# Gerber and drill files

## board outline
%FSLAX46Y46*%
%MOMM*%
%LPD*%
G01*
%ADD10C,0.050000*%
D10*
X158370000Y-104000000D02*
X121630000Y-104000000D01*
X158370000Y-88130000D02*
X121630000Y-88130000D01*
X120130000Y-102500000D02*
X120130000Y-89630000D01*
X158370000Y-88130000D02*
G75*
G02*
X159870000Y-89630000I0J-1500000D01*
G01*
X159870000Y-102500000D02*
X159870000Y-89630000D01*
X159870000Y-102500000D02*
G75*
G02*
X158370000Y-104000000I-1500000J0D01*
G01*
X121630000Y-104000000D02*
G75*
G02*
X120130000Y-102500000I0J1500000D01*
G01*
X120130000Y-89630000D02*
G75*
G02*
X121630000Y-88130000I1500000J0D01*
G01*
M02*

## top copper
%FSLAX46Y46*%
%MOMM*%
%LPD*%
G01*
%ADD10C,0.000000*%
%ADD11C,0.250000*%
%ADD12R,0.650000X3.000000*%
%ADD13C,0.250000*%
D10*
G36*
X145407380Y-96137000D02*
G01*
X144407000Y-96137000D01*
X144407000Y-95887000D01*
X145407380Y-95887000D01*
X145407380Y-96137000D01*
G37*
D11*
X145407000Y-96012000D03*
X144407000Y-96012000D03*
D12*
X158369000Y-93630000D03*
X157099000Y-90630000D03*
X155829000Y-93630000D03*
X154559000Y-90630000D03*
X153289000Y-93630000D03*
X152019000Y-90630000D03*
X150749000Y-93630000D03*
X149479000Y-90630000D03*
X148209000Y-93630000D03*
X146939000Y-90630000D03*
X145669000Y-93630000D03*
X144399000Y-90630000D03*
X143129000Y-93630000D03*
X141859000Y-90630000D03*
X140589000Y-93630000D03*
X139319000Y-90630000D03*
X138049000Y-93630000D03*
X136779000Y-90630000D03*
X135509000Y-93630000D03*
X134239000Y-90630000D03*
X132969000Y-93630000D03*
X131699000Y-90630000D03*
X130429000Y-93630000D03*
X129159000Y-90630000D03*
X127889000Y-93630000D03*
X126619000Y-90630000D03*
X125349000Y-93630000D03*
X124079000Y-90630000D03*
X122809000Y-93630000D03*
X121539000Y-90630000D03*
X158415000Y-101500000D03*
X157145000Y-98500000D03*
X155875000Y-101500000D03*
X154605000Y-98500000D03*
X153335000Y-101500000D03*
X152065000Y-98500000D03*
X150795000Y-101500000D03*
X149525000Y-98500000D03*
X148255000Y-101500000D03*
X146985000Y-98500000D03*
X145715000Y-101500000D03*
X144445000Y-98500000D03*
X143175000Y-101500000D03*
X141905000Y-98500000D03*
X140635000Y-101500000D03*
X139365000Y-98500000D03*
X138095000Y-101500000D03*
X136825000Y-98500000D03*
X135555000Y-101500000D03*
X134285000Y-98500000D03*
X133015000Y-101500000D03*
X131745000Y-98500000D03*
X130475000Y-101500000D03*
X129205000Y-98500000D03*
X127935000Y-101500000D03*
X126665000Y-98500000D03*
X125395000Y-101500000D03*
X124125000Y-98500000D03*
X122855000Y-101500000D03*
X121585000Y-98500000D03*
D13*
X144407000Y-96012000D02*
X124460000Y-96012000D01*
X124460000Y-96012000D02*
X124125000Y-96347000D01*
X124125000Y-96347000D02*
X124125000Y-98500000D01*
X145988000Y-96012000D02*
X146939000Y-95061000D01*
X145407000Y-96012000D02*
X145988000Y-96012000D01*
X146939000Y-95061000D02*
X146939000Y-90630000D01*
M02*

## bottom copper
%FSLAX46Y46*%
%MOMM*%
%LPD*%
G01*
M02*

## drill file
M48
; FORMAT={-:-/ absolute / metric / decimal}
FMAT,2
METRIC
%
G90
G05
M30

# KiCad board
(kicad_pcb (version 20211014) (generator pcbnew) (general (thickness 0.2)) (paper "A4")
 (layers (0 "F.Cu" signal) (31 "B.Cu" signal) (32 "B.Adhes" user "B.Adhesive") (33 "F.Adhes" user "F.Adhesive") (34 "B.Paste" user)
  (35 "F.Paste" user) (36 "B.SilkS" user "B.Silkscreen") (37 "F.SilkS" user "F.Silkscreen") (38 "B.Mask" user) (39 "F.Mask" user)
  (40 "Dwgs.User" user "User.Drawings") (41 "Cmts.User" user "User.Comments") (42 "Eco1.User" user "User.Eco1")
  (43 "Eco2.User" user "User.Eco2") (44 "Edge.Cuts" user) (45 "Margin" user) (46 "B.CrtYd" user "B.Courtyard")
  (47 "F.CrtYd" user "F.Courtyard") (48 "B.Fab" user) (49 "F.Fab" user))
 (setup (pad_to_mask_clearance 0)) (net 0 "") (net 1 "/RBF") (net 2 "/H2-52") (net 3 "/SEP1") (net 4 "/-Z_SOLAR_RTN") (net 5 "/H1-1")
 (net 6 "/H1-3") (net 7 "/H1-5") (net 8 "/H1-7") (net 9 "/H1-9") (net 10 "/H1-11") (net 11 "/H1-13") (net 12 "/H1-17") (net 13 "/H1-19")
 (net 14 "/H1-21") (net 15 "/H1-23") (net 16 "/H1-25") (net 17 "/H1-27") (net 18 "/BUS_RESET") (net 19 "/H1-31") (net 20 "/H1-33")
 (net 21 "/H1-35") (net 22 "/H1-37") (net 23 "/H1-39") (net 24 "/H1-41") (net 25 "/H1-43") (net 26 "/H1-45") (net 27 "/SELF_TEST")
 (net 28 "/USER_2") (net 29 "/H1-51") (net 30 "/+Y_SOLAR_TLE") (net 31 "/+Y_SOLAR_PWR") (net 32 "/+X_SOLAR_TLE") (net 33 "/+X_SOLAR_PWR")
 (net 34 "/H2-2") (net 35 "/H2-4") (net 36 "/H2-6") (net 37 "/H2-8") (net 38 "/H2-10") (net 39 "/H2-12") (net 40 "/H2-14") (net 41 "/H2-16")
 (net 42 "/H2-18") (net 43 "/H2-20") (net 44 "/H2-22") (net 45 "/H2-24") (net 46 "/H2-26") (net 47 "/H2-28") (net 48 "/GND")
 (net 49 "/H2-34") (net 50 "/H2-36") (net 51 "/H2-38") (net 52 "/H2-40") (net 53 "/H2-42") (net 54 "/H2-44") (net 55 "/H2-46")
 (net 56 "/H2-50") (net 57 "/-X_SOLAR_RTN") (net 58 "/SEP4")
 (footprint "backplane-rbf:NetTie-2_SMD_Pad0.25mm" (layer "F.Cu") (at 144.907 96.012 180)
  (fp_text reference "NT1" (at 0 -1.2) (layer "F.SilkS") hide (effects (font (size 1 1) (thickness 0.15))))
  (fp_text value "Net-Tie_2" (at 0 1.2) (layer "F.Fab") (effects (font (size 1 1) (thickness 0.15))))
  (fp_poly (pts (xy -0.50038 -0.125) (xy 0.5 -0.125) (xy 0.5 0.125) (xy -0.50038 0.125)) (layer "F.Cu") (width 0) (fill solid))
  (pad "1" smd circle locked (at -0.5 0 180) (size 0.25 0.25) (layers "F.Cu") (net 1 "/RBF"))
  (pad "2" smd circle locked (at 0.5 0 180) (size 0.25 0.25) (layers "F.Cu") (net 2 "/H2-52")))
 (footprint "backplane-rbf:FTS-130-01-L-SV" (layer "F.Cu") (at 139.954 92.13 -90)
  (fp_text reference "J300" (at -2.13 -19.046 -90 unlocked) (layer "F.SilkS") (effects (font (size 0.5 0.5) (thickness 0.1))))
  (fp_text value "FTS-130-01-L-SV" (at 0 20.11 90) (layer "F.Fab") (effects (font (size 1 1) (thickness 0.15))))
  (pad "1" smd rect locked (at 1.5 -18.415 270) (size 3 0.65) (layers "F.Cu" "F.Paste" "F.Mask") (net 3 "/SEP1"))
  (pad "2" smd rect locked (at -1.5 -17.145 270) (size 3 0.65) (layers "F.Cu" "F.Paste" "F.Mask") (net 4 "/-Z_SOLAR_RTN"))
  (pad "3" smd rect locked (at 1.5 -15.875 270) (size 3 0.65) (layers "F.Cu" "F.Paste" "F.Mask") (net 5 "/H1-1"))
  (pad "4" smd rect locked (at -1.5 -14.605 270) (size 3 0.65) (layers "F.Cu" "F.Paste" "F.Mask") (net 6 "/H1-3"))
  (pad "5" smd rect locked (at 1.5 -13.335 270) (size 3 0.65) (layers "F.Cu" "F.Paste" "F.Mask") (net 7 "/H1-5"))
  (pad "6" smd rect locked (at -1.5 -12.065 270) (size 3 0.65) (layers "F.Cu" "F.Paste" "F.Mask") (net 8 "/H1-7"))
  (pad "7" smd rect locked (at 1.5 -10.795 270) (size 3 0.65) (layers "F.Cu" "F.Paste" "F.Mask") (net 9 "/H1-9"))
  (pad "8" smd rect locked (at -1.5 -9.525 270) (size 3 0.65) (layers "F.Cu" "F.Paste" "F.Mask") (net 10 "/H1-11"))
  (pad "9" smd rect locked (at 1.5 -8.255 270) (size 3 0.65) (layers "F.Cu" "F.Paste" "F.Mask") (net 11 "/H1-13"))
  (pad "10" smd rect locked (at -1.5 -6.985 270) (size 3 0.65) (layers "F.Cu" "F.Paste" "F.Mask") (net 1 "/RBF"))
  (pad "11" smd rect locked (at 1.5 -5.715 270) (size 3 0.65) (layers "F.Cu" "F.Paste" "F.Mask") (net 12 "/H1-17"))
  (pad "12" smd rect locked (at -1.5 -4.445 270) (size 3 0.65) (layers "F.Cu" "F.Paste" "F.Mask") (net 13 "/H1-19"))
  (pad "13" smd rect locked (at 1.5 -3.175 270) (size 3 0.65) (layers "F.Cu" "F.Paste" "F.Mask") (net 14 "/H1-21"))
  (pad "14" smd rect locked (at -1.5 -1.905 270) (size 3 0.65) (layers "F.Cu" "F.Paste" "F.Mask") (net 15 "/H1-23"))
  (pad "15" smd rect locked (at 1.5 -0.635 270) (size 3 0.65) (layers "F.Cu" "F.Paste" "F.Mask") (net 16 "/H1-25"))
  (pad "16" smd rect locked (at -1.5 0.635 270) (size 3 0.65) (layers "F.Cu" "F.Paste" "F.Mask") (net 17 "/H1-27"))
  (pad "17" smd rect locked (at 1.5 1.905 270) (size 3 0.65) (layers "F.Cu" "F.Paste" "F.Mask") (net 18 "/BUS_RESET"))
  (pad "18" smd rect locked (at -1.5 3.175 270) (size 3 0.65) (layers "F.Cu" "F.Paste" "F.Mask") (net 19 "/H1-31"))
  (pad "19" smd rect locked (at 1.5 4.445 270) (size 3 0.65) (layers "F.Cu" "F.Paste" "F.Mask") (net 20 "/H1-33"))
  (pad "20" smd rect locked (at -1.5 5.715 270) (size 3 0.65) (layers "F.Cu" "F.Paste" "F.Mask") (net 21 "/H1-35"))
  (pad "21" smd rect locked (at 1.5 6.985 270) (size 3 0.65) (layers "F.Cu" "F.Paste" "F.Mask") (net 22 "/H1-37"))
  (pad "22" smd rect locked (at -1.5 8.255 270) (size 3 0.65) (layers "F.Cu" "F.Paste" "F.Mask") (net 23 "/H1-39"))
  (pad "23" smd rect locked (at 1.5 9.525 270) (size 3 0.65) (layers "F.Cu" "F.Paste" "F.Mask") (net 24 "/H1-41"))
  (pad "24" smd rect locked (at -1.5 10.795 270) (size 3 0.65) (layers "F.Cu" "F.Paste" "F.Mask") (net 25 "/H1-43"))
  (pad "25" smd rect locked (at 1.5 12.065 270) (size 3 0.65) (layers "F.Cu" "F.Paste" "F.Mask") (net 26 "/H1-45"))
  (pad "26" smd rect locked (at -1.5 13.335 270) (size 3 0.65) (layers "F.Cu" "F.Paste" "F.Mask") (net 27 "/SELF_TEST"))
  (pad "27" smd rect locked (at 1.5 14.605 270) (size 3 0.65) (layers "F.Cu" "F.Paste" "F.Mask") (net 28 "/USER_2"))
  (pad "28" smd rect locked (at -1.5 15.875 270) (size 3 0.65) (layers "F.Cu" "F.Paste" "F.Mask") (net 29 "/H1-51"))
  (pad "29" smd rect locked (at 1.5 17.145 270) (size 3 0.65) (layers "F.Cu" "F.Paste" "F.Mask") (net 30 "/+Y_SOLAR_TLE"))
  (pad "30" smd rect locked (at -1.5 18.415 270) (size 3 0.65) (layers "F.Cu" "F.Paste" "F.Mask") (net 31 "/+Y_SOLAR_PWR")))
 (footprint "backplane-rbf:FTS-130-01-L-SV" (layer "F.Cu") (at 140 100 -90)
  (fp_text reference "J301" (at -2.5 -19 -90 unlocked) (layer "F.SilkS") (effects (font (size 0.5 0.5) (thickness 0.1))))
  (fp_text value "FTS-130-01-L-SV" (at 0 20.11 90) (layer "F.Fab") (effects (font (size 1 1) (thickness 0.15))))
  (pad "1" smd rect locked (at 1.5 -18.415 270) (size 3 0.65) (layers "F.Cu" "F.Paste" "F.Mask") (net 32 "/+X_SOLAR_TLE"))
  (pad "2" smd rect locked (at -1.5 -17.145 270) (size 3 0.65) (layers "F.Cu" "F.Paste" "F.Mask") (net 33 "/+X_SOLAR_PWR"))
  (pad "3" smd rect locked (at 1.5 -15.875 270) (size 3 0.65) (layers "F.Cu" "F.Paste" "F.Mask") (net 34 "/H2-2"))
  (pad "4" smd rect locked (at -1.5 -14.605 270) (size 3 0.65) (layers "F.Cu" "F.Paste" "F.Mask") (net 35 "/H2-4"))
  (pad "5" smd rect locked (at 1.5 -13.335 270) (size 3 0.65) (layers "F.Cu" "F.Paste" "F.Mask") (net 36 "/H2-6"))
  (pad "6" smd rect locked (at -1.5 -12.065 270) (size 3 0.65) (layers "F.Cu" "F.Paste" "F.Mask") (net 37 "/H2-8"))
  (pad "7" smd rect locked (at 1.5 -10.795 270) (size 3 0.65) (layers "F.Cu" "F.Paste" "F.Mask") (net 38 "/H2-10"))
  (pad "8" smd rect locked (at -1.5 -9.525 270) (size 3 0.65) (layers "F.Cu" "F.Paste" "F.Mask") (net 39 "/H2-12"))
  (pad "9" smd rect locked (at 1.5 -8.255 270) (size 3 0.65) (layers "F.Cu" "F.Paste" "F.Mask") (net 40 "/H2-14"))
  (pad "10" smd rect locked (at -1.5 -6.985 270) (size 3 0.65) (layers "F.Cu" "F.Paste" "F.Mask") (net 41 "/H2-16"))
  (pad "11" smd rect locked (at 1.5 -5.715 270) (size 3 0.65) (layers "F.Cu" "F.Paste" "F.Mask") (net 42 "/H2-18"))
  (pad "12" smd rect locked (at -1.5 -4.445 270) (size 3 0.65) (layers "F.Cu" "F.Paste" "F.Mask") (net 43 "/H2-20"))
  (pad "13" smd rect locked (at 1.5 -3.175 270) (size 3 0.65) (layers "F.Cu" "F.Paste" "F.Mask") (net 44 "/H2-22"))
  (pad "14" smd rect locked (at -1.5 -1.905 270) (size 3 0.65) (layers "F.Cu" "F.Paste" "F.Mask") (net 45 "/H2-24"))
  (pad "15" smd rect locked (at 1.5 -0.635 270) (size 3 0.65) (layers "F.Cu" "F.Paste" "F.Mask") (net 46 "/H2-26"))
  (pad "16" smd rect locked (at -1.5 0.635 270) (size 3 0.65) (layers "F.Cu" "F.Paste" "F.Mask") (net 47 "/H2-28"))
  (pad "17" smd rect locked (at 1.5 1.905 270) (size 3 0.65) (layers "F.Cu" "F.Paste" "F.Mask") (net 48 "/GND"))
  (pad "18" smd rect locked (at -1.5 3.175 270) (size 3 0.65) (layers "F.Cu" "F.Paste" "F.Mask") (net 48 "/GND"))
  (pad "19" smd rect locked (at 1.5 4.445 270) (size 3 0.65) (layers "F.Cu" "F.Paste" "F.Mask") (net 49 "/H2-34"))
  (pad "20" smd rect locked (at -1.5 5.715 270) (size 3 0.65) (layers "F.Cu" "F.Paste" "F.Mask") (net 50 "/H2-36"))
  (pad "21" smd rect locked (at 1.5 6.985 270) (size 3 0.65) (layers "F.Cu" "F.Paste" "F.Mask") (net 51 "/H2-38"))
  (pad "22" smd rect locked (at -1.5 8.255 270) (size 3 0.65) (layers "F.Cu" "F.Paste" "F.Mask") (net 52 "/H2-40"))
  (pad "23" smd rect locked (at 1.5 9.525 270) (size 3 0.65) (layers "F.Cu" "F.Paste" "F.Mask") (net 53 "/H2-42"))
  (pad "24" smd rect locked (at -1.5 10.795 270) (size 3 0.65) (layers "F.Cu" "F.Paste" "F.Mask") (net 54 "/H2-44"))
  (pad "25" smd rect locked (at 1.5 12.065 270) (size 3 0.65) (layers "F.Cu" "F.Paste" "F.Mask") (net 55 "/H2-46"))
  (pad "26" smd rect locked (at -1.5 13.335 270) (size 3 0.65) (layers "F.Cu" "F.Paste" "F.Mask") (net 48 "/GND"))
  (pad "27" smd rect locked (at 1.5 14.605 270) (size 3 0.65) (layers "F.Cu" "F.Paste" "F.Mask") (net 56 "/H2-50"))
  (pad "28" smd rect locked (at -1.5 15.875 270) (size 3 0.65) (layers "F.Cu" "F.Paste" "F.Mask") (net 2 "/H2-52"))
  (pad "29" smd rect locked (at 1.5 17.145 270) (size 3 0.65) (layers "F.Cu" "F.Paste" "F.Mask") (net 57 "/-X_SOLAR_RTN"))
  (pad "30" smd rect locked (at -1.5 18.415 270) (size 3 0.65) (layers "F.Cu" "F.Paste" "F.Mask") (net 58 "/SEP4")))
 (gr_line (start 158.37 104) (end 121.63 104) (layer "Edge.Cuts") (width 0.05))
 (gr_line (start 158.37 88.13) (end 121.63 88.13) (layer "Edge.Cuts") (width 0.05))
 (gr_line (start 120.13 102.5) (end 120.13 89.63) (layer "Edge.Cuts") (width 0.05))
 (gr_arc (start 158.37 88.13) (mid 159.43066 88.56934) (end 159.87 89.63) (layer "Edge.Cuts") (width 0.05))
 (gr_line (start 159.87 102.5) (end 159.87 89.63) (layer "Edge.Cuts") (width 0.05))
 (gr_arc (start 159.87 102.5) (mid 159.43066 103.56066) (end 158.37 104) (layer "Edge.Cuts") (width 0.05))
 (gr_arc (start 121.63 104) (mid 120.56934 103.56066) (end 120.13 102.5) (layer "Edge.Cuts") (width 0.05))
 (gr_arc (start 120.13 89.63) (mid 120.56934 88.56934) (end 121.63 88.13) (layer "Edge.Cuts") (width 0.05))
 (segment (start 144.407 96.012) (end 124.46 96.012) (width 0.25) (layer "F.Cu") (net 2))
 (segment (start 124.46 96.012) (end 124.125 96.347) (width 0.25) (layer "F.Cu") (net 2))
 (segment (start 124.125 96.347) (end 124.125 98.5) (width 0.25) (layer "F.Cu") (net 2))
 (segment (start 145.988 96.012) (end 146.939 95.061) (width 0.25) (layer "F.Cu") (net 1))
 (segment (start 145.407 96.012) (end 145.988 96.012) (width 0.25) (layer "F.Cu") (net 1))
 (segment (start 146.939 95.061) (end 146.939 90.63) (width 0.25) (layer "F.Cu") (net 1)))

